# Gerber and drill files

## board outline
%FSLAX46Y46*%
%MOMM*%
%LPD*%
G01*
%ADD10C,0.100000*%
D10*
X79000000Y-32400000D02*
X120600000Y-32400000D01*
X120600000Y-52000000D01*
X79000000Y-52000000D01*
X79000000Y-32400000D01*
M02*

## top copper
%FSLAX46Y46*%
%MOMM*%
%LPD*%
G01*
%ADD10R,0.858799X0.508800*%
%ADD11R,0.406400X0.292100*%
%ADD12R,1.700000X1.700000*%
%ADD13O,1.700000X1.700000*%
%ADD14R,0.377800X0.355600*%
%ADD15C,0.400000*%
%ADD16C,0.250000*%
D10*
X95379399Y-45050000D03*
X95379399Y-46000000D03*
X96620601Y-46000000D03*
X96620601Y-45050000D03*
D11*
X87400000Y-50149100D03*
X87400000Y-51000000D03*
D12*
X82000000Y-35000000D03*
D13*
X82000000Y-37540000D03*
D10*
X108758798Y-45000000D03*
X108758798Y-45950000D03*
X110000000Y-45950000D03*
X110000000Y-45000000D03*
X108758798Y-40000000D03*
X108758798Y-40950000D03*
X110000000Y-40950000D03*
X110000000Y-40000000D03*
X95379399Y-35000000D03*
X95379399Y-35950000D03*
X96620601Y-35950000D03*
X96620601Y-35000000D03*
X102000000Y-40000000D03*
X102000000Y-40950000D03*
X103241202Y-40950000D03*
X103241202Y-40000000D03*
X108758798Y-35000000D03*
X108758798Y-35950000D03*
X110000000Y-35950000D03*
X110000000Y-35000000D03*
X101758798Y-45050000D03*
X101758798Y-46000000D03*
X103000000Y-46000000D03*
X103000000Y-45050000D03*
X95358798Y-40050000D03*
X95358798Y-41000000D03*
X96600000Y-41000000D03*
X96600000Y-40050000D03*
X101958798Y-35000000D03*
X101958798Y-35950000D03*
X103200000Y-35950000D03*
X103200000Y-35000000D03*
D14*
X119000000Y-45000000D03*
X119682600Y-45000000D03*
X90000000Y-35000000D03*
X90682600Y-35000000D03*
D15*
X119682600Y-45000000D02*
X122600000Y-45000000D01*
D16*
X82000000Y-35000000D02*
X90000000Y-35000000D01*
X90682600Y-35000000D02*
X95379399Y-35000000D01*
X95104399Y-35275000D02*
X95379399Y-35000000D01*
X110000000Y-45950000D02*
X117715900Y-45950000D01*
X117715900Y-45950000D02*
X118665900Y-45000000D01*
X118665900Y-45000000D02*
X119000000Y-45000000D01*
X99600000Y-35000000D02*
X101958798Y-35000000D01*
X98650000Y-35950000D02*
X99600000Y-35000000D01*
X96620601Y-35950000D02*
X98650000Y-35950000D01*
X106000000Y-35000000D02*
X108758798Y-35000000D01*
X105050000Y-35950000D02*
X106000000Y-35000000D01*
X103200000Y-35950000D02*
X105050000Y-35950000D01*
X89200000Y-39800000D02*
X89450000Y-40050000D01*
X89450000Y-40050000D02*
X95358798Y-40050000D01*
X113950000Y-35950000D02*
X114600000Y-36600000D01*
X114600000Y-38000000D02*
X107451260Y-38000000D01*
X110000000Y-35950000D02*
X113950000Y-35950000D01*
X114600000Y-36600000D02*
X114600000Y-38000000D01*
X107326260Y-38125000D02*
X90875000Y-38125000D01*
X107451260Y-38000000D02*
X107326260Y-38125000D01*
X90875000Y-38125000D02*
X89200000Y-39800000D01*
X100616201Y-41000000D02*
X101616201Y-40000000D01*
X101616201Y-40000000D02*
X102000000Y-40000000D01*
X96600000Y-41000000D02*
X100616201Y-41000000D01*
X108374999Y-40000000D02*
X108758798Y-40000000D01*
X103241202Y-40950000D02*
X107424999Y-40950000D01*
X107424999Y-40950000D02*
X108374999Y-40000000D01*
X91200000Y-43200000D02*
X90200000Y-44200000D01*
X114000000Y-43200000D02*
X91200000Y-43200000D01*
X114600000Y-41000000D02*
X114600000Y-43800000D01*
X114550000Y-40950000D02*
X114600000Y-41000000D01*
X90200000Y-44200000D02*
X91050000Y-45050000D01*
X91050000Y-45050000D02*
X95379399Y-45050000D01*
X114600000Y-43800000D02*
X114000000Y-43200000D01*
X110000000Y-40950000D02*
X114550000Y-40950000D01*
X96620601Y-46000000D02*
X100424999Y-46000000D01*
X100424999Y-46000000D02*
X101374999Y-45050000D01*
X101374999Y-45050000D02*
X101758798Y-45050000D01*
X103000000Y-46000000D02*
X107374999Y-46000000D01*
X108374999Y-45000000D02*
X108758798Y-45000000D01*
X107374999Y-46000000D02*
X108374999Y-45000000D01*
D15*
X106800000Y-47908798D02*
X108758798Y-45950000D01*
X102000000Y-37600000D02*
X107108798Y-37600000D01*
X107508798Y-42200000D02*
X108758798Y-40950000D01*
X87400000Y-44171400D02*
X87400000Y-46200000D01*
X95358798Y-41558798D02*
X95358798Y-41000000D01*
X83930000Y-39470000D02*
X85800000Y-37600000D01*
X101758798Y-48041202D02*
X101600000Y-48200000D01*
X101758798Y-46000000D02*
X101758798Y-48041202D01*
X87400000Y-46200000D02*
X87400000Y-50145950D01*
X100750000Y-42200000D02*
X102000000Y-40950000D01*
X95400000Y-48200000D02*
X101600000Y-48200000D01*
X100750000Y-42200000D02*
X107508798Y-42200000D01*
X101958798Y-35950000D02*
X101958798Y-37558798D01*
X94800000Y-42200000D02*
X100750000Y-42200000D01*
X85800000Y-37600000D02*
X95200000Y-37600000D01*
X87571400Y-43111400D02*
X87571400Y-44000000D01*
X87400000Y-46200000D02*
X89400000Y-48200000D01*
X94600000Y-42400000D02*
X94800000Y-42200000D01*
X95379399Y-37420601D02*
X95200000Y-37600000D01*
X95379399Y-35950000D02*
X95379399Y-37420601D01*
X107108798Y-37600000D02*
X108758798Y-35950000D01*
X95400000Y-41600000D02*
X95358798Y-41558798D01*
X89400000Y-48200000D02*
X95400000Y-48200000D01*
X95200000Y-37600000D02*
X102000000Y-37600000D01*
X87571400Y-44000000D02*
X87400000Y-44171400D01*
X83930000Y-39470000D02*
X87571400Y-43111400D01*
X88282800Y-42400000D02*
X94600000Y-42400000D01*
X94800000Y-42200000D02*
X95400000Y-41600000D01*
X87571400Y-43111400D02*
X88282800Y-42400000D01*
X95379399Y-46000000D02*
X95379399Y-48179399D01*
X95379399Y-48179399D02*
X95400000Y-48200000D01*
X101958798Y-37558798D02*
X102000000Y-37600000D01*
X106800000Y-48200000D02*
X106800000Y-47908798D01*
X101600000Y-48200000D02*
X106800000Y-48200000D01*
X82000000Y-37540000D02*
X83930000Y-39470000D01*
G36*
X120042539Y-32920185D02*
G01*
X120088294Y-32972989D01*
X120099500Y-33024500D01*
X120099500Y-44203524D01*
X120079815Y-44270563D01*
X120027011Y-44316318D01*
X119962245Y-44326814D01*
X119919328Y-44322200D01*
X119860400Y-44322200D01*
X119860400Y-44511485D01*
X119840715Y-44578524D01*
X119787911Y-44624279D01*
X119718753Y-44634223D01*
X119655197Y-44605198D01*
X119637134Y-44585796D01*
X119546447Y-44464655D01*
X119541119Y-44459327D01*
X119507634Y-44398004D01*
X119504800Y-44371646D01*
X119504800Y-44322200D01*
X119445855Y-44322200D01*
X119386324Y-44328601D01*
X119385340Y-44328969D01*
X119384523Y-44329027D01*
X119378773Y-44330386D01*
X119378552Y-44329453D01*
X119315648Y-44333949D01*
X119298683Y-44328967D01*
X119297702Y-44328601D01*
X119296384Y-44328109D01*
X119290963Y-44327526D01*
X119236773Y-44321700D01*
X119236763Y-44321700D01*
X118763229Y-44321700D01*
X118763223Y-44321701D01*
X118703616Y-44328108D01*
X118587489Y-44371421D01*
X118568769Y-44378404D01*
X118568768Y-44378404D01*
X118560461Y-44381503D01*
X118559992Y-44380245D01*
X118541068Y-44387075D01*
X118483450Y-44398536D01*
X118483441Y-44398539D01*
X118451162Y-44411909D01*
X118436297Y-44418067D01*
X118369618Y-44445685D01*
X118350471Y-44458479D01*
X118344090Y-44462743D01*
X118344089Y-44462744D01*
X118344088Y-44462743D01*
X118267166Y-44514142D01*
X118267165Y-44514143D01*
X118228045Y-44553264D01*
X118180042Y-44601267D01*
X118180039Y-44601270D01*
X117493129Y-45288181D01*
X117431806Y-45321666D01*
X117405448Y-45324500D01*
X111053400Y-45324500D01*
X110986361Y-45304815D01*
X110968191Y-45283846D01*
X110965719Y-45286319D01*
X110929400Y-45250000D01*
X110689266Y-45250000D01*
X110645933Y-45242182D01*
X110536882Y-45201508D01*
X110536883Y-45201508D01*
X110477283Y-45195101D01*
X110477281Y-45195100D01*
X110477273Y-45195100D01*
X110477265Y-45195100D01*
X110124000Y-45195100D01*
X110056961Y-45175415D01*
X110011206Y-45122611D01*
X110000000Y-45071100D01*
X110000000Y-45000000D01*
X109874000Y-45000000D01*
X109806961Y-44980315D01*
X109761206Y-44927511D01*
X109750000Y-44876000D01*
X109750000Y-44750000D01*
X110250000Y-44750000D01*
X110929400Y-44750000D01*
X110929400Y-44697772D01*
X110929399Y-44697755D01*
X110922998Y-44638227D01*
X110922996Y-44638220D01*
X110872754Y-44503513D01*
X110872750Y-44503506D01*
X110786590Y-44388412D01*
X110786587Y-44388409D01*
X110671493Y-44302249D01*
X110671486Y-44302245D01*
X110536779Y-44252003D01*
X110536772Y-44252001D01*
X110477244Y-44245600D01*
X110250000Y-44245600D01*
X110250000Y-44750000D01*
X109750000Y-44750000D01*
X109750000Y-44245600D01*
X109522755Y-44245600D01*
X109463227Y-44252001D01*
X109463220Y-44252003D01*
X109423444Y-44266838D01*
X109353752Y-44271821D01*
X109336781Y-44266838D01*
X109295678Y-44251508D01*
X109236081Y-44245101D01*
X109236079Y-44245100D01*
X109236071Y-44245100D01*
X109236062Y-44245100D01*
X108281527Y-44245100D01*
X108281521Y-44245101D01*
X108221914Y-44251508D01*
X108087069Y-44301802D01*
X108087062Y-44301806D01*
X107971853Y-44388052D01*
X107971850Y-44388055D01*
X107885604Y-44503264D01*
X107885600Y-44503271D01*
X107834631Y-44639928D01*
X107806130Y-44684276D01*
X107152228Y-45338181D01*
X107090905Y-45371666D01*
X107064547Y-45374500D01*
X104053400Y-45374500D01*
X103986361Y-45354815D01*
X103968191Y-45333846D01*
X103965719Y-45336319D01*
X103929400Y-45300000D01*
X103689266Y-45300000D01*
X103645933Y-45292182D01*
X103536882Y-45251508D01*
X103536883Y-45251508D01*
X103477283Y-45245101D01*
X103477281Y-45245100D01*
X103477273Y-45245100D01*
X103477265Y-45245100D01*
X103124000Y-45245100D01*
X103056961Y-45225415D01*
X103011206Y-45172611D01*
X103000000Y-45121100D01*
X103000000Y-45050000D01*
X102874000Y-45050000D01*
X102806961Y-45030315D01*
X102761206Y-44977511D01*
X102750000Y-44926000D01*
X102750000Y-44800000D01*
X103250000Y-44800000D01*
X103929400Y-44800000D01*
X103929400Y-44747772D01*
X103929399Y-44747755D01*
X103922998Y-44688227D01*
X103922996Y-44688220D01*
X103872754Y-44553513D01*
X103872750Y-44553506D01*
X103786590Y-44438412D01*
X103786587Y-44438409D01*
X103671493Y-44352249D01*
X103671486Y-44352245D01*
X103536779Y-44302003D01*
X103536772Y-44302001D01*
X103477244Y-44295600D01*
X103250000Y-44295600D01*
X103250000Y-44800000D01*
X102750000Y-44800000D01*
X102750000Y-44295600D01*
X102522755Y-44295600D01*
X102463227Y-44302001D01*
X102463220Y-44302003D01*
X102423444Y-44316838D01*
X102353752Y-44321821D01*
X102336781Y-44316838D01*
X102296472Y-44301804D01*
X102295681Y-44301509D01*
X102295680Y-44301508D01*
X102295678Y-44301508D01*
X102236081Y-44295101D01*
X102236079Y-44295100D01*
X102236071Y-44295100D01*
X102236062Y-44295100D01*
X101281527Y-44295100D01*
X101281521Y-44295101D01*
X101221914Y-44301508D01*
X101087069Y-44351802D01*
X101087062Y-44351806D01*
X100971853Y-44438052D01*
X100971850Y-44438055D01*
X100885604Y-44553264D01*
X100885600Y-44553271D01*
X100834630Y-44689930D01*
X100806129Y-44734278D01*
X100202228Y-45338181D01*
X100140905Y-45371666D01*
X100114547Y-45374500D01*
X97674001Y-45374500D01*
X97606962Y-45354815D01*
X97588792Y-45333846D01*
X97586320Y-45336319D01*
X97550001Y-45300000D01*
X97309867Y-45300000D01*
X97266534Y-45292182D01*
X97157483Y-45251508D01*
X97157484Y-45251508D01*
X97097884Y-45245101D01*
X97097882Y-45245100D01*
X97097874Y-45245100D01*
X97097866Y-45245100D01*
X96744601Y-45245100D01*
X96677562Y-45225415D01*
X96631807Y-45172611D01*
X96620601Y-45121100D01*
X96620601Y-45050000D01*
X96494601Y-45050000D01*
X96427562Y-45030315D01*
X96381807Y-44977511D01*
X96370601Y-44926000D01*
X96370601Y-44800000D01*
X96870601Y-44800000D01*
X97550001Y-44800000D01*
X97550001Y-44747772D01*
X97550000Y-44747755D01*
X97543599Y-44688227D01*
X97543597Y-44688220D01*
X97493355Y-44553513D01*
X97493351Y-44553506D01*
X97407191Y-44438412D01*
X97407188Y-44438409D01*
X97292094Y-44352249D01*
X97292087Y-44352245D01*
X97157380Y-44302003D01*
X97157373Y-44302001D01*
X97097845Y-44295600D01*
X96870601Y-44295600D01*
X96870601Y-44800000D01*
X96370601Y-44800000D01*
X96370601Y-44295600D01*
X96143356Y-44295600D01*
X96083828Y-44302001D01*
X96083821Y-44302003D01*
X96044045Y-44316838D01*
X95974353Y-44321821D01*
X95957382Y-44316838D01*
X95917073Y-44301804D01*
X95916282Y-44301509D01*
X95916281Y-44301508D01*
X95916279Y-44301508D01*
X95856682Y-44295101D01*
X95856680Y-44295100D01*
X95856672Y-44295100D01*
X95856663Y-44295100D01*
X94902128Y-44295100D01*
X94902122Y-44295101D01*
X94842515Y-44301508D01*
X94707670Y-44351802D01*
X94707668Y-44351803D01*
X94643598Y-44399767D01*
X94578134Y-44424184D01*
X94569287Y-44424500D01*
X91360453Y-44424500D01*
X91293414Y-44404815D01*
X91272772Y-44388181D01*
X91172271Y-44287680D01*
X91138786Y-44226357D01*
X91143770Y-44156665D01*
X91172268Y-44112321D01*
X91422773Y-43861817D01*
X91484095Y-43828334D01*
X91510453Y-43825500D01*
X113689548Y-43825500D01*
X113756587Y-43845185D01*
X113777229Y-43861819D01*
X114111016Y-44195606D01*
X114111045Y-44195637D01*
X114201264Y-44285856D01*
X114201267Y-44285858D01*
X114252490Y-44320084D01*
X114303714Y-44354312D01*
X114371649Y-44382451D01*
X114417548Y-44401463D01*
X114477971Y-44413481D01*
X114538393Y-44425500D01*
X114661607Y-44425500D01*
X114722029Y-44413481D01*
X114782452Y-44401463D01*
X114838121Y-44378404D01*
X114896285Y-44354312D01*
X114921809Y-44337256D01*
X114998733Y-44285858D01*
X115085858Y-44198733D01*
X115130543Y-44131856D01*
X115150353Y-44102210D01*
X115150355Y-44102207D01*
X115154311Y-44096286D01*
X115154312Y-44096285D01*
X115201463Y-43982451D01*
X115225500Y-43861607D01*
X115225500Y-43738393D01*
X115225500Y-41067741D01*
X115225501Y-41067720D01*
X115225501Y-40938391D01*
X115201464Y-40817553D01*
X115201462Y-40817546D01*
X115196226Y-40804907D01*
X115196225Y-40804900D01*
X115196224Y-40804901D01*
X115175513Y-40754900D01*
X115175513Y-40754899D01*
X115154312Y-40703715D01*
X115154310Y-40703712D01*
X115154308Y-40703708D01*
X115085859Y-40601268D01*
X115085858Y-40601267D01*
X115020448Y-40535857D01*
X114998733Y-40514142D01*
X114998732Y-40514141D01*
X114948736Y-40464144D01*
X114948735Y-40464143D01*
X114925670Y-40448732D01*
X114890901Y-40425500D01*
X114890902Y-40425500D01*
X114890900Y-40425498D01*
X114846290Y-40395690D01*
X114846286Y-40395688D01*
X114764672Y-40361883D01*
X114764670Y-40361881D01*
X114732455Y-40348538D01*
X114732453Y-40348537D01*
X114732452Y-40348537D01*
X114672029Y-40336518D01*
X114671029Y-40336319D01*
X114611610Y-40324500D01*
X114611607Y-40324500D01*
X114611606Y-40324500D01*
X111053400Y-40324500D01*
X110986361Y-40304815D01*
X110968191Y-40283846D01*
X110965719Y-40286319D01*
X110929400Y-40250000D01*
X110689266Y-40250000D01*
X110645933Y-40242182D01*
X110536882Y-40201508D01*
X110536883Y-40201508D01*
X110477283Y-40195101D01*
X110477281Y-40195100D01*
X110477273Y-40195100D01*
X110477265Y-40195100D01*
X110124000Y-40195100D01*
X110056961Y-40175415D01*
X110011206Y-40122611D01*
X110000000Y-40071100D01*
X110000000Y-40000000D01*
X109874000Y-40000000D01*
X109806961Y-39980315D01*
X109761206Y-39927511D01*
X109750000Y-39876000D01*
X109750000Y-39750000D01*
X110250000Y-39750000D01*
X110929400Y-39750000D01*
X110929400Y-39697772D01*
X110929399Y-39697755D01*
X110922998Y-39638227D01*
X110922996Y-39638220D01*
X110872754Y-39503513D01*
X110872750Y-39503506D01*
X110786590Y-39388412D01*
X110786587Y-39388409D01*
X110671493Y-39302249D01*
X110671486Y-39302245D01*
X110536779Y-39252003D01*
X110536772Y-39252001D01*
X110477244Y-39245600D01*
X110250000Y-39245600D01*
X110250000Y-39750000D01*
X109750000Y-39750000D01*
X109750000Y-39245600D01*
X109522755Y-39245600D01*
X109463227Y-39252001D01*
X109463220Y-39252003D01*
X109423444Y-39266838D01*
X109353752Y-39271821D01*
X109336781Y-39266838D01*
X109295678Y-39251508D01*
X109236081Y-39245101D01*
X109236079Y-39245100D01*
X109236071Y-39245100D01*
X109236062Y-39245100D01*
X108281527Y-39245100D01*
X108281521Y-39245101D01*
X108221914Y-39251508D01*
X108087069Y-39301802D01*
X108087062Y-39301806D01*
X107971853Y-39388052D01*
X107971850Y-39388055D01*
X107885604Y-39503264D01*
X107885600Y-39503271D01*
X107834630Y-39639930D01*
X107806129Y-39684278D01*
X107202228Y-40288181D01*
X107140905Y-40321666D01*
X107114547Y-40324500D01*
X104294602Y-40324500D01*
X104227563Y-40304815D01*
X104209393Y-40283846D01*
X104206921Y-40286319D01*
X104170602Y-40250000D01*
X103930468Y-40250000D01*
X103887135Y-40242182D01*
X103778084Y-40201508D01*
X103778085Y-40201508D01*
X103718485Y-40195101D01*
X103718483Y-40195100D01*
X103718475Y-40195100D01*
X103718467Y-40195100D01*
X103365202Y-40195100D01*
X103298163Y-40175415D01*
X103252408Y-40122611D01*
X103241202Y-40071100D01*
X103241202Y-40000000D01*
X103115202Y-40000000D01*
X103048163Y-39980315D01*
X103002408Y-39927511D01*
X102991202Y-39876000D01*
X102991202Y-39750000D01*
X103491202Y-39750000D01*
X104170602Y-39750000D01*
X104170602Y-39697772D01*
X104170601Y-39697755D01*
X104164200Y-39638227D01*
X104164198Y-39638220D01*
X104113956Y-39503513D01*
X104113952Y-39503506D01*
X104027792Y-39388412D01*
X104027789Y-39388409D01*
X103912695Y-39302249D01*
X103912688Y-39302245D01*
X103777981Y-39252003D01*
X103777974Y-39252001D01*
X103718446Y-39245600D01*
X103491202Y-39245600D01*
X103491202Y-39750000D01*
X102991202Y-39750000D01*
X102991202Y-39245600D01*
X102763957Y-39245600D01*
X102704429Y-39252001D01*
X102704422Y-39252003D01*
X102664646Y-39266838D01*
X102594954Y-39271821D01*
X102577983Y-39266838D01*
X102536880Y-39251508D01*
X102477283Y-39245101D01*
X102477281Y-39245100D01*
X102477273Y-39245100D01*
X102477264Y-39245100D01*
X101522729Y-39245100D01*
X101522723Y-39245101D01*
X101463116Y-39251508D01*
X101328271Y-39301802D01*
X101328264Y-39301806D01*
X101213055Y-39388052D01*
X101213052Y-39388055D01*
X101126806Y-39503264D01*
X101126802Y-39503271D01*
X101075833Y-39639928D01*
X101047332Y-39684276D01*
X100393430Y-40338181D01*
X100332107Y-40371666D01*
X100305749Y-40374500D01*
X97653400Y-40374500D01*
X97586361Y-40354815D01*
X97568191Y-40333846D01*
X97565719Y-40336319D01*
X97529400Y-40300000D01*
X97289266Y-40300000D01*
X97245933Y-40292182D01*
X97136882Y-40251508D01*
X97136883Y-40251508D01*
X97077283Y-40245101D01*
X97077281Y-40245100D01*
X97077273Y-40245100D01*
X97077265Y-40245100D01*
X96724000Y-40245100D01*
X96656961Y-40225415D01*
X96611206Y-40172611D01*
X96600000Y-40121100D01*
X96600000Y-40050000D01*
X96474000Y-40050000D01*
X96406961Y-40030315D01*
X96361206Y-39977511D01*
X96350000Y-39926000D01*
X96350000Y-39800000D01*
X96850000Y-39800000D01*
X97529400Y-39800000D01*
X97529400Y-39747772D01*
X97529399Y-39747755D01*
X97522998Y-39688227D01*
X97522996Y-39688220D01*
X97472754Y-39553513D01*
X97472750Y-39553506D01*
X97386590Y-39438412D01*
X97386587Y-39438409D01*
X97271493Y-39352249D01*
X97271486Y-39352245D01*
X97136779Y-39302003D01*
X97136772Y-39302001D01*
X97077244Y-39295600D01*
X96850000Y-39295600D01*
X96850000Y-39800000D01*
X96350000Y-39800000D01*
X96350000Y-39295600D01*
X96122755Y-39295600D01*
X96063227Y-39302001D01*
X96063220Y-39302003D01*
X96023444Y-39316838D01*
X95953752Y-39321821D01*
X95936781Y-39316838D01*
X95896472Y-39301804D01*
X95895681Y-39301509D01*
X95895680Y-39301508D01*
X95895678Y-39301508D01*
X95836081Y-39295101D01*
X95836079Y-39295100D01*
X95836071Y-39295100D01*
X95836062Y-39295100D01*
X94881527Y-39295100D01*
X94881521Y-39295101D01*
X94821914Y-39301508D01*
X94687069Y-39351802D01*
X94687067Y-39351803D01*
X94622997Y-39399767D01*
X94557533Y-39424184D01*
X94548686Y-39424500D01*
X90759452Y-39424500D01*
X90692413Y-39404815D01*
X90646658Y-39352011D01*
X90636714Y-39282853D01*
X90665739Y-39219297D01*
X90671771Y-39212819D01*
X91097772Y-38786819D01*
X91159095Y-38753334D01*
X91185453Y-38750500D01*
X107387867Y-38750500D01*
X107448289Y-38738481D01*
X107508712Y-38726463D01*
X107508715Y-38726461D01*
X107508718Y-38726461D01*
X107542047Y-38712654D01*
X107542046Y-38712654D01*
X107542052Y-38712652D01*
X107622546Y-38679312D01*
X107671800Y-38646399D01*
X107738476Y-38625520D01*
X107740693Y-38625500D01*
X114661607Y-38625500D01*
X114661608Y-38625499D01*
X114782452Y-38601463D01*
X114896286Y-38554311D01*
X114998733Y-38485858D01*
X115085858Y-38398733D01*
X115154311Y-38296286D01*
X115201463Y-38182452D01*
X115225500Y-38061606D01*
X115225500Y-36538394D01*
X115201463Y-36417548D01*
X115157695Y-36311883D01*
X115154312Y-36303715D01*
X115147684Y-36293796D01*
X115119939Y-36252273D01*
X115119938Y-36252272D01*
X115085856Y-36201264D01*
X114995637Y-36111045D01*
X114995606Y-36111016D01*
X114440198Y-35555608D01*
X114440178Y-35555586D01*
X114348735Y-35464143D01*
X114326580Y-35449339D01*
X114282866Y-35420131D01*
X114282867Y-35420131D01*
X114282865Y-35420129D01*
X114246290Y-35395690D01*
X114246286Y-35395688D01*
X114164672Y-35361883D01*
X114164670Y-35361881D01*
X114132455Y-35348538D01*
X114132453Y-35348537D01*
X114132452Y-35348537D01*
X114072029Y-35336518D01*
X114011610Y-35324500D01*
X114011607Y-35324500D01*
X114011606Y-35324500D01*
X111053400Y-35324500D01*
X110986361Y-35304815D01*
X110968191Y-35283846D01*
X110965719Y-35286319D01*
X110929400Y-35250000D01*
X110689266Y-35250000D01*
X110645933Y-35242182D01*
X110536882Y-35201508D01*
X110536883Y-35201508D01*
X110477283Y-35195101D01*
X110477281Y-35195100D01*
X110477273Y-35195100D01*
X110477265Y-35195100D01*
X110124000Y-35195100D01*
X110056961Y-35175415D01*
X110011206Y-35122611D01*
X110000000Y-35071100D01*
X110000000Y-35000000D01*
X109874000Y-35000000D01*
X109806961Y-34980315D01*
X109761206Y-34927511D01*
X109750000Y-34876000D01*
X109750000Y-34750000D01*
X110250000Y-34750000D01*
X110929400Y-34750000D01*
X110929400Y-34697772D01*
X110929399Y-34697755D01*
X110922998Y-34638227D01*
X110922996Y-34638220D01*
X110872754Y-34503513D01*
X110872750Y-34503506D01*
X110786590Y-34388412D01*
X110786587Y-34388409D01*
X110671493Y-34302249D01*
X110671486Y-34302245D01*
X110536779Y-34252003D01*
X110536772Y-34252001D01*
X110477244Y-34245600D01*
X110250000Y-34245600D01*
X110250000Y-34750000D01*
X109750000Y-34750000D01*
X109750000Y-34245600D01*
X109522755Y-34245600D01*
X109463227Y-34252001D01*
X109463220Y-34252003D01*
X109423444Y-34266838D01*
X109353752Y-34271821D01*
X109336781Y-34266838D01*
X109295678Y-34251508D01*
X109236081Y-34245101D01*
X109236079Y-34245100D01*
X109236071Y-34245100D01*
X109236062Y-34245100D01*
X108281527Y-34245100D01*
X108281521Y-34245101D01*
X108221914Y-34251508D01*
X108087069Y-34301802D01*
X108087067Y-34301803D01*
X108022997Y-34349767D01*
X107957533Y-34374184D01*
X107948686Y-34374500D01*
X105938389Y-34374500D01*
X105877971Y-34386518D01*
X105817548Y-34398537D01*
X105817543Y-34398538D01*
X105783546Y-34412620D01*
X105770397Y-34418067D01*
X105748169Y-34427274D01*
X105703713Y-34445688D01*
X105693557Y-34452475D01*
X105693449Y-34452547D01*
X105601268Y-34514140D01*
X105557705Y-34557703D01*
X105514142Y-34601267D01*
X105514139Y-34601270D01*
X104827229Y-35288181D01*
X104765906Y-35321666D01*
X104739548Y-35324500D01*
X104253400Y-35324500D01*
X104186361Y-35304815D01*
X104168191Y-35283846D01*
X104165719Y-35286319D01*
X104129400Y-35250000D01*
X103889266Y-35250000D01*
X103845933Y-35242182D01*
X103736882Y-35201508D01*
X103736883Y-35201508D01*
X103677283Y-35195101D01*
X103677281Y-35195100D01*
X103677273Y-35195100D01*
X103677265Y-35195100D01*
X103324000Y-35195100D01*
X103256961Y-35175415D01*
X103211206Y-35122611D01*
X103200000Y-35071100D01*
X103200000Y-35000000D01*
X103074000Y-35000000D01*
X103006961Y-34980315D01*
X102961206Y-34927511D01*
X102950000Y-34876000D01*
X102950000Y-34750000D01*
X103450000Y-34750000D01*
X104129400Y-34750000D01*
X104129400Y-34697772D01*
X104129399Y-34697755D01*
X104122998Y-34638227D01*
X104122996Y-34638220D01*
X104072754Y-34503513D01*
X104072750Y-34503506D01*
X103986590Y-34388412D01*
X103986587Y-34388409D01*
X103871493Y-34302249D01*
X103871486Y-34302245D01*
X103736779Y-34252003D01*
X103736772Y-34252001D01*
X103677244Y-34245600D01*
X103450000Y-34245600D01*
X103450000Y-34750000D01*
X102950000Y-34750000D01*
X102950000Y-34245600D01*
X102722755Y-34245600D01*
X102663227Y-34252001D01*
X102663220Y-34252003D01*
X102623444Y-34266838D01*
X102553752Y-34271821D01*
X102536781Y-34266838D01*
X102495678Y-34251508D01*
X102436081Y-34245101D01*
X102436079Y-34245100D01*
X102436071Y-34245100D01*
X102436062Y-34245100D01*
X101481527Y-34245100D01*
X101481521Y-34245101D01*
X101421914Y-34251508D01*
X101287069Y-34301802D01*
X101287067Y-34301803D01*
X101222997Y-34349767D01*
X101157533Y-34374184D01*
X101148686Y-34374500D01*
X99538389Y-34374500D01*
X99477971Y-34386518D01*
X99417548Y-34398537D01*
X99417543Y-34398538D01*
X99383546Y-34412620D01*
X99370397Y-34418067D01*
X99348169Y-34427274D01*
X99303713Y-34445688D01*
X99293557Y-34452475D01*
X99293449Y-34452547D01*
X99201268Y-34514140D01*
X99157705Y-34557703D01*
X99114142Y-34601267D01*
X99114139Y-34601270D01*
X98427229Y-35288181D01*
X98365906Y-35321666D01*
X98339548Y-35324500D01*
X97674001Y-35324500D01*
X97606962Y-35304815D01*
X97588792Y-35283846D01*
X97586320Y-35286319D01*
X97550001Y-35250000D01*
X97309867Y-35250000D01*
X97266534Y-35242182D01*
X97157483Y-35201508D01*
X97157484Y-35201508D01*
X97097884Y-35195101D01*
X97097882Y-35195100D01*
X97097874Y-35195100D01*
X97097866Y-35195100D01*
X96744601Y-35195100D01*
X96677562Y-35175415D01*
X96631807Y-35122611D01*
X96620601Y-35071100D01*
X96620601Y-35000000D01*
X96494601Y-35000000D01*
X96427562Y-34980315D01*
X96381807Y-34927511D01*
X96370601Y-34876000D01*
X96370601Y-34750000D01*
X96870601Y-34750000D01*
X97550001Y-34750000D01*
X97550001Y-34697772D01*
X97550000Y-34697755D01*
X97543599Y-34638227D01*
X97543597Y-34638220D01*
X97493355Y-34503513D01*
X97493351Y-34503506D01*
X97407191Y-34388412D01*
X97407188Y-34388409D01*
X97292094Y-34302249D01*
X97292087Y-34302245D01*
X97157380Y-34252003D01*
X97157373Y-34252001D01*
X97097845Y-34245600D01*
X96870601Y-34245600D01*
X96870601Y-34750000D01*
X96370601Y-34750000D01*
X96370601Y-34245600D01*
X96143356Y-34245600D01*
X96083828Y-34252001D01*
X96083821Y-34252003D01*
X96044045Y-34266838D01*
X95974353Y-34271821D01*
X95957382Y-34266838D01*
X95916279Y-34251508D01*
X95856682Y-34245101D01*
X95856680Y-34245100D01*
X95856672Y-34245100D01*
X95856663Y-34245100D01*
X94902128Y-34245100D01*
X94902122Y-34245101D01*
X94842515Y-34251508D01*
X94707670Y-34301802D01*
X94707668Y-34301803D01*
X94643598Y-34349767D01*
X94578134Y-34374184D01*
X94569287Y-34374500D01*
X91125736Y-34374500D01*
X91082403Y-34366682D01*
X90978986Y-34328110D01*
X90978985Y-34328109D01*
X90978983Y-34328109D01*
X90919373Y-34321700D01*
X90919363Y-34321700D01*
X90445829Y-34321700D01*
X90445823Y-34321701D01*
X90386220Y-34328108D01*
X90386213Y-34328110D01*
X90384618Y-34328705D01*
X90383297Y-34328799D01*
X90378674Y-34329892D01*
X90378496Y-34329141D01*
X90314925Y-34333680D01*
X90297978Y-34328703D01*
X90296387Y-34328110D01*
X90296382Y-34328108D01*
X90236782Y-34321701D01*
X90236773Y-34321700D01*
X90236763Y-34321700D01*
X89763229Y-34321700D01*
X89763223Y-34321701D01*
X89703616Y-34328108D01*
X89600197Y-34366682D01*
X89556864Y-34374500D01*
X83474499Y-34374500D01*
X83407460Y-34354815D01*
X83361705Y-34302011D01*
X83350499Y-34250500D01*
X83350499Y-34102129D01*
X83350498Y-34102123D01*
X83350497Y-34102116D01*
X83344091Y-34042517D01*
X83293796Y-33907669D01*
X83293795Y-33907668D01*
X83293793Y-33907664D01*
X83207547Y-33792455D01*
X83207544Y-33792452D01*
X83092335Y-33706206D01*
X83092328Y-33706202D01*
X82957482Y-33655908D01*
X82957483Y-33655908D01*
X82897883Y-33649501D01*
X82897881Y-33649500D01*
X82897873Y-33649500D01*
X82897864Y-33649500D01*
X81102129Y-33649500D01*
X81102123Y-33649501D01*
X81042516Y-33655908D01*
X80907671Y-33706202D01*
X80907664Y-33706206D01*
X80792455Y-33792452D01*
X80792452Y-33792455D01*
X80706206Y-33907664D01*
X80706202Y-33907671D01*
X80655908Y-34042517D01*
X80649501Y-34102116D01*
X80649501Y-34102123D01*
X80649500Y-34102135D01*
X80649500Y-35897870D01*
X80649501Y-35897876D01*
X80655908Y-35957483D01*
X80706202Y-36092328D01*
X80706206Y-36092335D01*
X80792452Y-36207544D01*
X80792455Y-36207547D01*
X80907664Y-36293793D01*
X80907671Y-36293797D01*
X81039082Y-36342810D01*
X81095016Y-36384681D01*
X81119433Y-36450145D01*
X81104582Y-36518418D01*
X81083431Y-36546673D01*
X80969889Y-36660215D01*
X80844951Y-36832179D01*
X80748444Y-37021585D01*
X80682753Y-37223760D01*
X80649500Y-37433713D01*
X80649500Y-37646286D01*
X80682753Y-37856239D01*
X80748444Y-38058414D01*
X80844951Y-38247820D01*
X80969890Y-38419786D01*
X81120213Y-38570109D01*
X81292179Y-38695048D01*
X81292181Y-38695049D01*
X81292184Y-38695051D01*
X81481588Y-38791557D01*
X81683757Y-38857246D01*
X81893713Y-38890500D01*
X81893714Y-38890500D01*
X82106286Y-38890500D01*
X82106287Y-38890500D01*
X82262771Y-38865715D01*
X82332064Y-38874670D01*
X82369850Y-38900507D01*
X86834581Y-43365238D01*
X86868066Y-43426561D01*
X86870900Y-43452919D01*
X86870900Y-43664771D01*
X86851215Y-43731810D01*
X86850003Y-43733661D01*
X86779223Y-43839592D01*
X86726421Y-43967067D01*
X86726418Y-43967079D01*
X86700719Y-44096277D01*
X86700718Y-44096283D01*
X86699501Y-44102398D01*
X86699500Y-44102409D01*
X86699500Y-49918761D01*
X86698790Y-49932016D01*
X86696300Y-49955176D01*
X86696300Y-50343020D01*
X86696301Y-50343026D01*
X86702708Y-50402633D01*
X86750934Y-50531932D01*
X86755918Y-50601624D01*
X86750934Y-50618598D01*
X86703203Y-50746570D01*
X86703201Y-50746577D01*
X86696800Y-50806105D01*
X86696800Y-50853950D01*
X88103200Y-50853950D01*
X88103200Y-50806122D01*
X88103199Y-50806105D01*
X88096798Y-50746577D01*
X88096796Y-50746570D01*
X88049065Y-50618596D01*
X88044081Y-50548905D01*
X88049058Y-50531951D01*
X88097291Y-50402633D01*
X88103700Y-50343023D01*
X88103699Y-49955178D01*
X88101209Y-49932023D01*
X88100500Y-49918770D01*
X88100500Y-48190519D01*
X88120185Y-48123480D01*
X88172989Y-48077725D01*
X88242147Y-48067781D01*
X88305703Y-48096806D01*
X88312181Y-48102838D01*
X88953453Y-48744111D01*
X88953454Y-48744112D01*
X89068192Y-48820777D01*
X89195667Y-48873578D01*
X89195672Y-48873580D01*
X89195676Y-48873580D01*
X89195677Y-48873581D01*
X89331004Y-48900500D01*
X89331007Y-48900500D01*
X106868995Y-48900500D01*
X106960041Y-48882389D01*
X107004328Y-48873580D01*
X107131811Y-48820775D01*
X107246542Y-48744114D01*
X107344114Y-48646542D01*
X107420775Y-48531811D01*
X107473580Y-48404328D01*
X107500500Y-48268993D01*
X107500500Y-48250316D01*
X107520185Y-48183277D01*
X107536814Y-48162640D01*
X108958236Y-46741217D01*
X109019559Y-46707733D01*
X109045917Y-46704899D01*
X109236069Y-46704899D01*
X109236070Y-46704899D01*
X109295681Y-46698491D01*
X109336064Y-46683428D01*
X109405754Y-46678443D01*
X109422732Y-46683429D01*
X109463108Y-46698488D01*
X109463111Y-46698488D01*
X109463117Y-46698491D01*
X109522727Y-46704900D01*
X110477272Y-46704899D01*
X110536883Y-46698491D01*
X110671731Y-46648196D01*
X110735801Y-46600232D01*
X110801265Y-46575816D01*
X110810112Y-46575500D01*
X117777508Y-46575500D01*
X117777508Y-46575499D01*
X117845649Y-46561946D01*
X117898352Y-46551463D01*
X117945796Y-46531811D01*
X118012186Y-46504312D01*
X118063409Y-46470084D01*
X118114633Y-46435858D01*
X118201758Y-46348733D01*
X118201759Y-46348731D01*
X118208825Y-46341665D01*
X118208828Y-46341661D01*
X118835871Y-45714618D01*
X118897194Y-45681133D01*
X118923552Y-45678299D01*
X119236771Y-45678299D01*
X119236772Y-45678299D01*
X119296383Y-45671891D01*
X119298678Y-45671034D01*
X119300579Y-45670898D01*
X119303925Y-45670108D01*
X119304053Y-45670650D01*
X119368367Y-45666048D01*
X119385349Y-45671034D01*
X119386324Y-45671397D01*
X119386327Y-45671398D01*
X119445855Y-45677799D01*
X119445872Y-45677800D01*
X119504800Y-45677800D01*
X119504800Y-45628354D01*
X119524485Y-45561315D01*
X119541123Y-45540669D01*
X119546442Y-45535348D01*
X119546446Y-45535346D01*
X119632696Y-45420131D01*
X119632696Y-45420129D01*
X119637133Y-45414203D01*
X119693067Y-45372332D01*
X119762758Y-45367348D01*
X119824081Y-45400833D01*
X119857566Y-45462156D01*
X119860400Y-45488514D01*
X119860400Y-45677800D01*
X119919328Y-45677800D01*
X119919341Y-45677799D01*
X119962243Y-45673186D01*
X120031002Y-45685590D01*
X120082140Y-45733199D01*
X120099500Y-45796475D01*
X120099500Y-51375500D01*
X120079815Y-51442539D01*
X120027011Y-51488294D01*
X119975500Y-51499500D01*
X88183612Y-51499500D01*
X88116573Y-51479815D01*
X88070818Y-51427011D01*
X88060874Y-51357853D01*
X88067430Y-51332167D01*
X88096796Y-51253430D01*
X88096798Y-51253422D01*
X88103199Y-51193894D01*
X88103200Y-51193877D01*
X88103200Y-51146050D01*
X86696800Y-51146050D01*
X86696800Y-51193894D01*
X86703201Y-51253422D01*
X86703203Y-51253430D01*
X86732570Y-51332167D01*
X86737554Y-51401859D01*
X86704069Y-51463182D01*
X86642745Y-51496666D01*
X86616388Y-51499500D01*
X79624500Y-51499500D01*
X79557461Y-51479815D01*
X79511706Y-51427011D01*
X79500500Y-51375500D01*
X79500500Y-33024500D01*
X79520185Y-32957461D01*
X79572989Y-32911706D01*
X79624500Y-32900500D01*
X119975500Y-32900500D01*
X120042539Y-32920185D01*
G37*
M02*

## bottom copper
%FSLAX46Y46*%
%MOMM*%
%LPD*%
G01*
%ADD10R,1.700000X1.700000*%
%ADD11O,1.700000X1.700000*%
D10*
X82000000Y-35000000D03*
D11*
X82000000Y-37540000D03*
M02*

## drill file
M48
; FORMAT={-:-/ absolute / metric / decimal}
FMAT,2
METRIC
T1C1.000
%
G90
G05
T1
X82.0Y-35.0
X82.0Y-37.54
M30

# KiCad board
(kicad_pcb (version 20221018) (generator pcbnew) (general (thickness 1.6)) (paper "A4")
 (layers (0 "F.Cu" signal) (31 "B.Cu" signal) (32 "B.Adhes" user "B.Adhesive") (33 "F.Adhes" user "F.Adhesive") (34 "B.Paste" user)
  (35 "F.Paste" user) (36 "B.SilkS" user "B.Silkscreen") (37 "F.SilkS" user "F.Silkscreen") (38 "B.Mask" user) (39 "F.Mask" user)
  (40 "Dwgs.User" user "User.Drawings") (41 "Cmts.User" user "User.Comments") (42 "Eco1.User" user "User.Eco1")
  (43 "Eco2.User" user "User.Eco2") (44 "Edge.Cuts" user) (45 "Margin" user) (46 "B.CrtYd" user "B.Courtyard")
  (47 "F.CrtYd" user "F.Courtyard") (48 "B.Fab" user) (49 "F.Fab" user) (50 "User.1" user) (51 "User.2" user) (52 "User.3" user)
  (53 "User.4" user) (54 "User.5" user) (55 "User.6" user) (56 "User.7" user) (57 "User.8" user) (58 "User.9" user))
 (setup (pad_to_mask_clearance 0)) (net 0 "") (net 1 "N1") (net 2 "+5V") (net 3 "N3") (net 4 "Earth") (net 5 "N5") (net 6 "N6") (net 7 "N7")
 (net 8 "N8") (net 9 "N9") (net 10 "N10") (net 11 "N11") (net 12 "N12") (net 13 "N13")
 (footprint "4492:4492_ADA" (layer "F.Cu") (at 96 45.525)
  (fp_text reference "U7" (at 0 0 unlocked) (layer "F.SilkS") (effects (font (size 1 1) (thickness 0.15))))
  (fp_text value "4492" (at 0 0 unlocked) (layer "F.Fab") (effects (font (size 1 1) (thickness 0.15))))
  (pad "1" smd rect (at -0.620601 -0.475) (size 0.858799 0.5088) (layers "F.Cu" "F.Paste" "F.Mask") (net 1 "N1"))
  (pad "2" smd rect (at -0.620601 0.475) (size 0.858799 0.5088) (layers "F.Cu" "F.Paste" "F.Mask") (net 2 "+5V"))
  (pad "3" smd rect (at 0.620601 0.475) (size 0.858799 0.5088) (layers "F.Cu" "F.Paste" "F.Mask") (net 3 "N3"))
  (pad "4" smd rect (at 0.620601 -0.475) (size 0.858799 0.5088) (layers "F.Cu" "F.Paste" "F.Mask") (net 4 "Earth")))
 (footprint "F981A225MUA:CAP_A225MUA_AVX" (layer "F.Cu") (at 87.4 50.57455 -90)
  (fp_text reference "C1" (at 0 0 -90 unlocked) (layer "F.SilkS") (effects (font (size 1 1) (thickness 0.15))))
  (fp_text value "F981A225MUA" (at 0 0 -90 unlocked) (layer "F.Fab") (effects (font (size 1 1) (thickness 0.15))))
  (pad "1" smd rect (at -0.42545 0 270) (size 0.2921 0.4064) (layers "F.Cu" "F.Paste" "F.Mask") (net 2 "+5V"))
  (pad "2" smd rect (at 0.42545 0 270) (size 0.2921 0.4064) (layers "F.Cu" "F.Paste" "F.Mask") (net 4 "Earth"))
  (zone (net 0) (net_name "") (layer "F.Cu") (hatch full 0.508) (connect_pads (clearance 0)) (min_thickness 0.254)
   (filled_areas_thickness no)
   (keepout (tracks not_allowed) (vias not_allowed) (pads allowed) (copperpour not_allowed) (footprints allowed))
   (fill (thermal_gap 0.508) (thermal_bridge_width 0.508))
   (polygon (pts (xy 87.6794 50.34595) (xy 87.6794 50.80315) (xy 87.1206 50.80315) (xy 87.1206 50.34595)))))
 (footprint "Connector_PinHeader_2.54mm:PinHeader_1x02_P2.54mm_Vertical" (layer "F.Cu") (at 82 35)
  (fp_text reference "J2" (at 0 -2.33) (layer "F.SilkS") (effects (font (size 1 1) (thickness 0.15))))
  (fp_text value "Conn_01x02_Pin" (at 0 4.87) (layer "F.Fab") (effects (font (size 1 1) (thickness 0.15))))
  (pad "1" thru_hole rect (at 0 0) (size 1.7 1.7) (drill 1) (layers "*.Cu" "*.Mask") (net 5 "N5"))
  (pad "2" thru_hole oval (at 0 2.54) (size 1.7 1.7) (drill 1) (layers "*.Cu" "*.Mask") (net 2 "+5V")))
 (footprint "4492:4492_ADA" (layer "F.Cu") (at 109.379399 45.475)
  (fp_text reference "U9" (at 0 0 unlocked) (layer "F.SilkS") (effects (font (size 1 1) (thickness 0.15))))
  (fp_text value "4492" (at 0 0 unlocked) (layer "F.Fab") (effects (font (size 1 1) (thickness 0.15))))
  (pad "1" smd rect (at -0.620601 -0.475) (size 0.858799 0.5088) (layers "F.Cu" "F.Paste" "F.Mask") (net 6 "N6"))
  (pad "2" smd rect (at -0.620601 0.475) (size 0.858799 0.5088) (layers "F.Cu" "F.Paste" "F.Mask") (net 2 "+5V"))
  (pad "3" smd rect (at 0.620601 0.475) (size 0.858799 0.5088) (layers "F.Cu" "F.Paste" "F.Mask") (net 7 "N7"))
  (pad "4" smd rect (at 0.620601 -0.475) (size 0.858799 0.5088) (layers "F.Cu" "F.Paste" "F.Mask") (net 4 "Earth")))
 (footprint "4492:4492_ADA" (layer "F.Cu") (at 109.379399 40.475)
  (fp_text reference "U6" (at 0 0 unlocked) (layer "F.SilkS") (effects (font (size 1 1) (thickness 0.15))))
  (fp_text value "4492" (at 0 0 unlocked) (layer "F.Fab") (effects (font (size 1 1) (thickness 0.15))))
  (pad "1" smd rect (at -0.620601 -0.475) (size 0.858799 0.5088) (layers "F.Cu" "F.Paste" "F.Mask") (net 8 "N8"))
  (pad "2" smd rect (at -0.620601 0.475) (size 0.858799 0.5088) (layers "F.Cu" "F.Paste" "F.Mask") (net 2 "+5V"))
  (pad "3" smd rect (at 0.620601 0.475) (size 0.858799 0.5088) (layers "F.Cu" "F.Paste" "F.Mask") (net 1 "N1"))
  (pad "4" smd rect (at 0.620601 -0.475) (size 0.858799 0.5088) (layers "F.Cu" "F.Paste" "F.Mask") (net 4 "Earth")))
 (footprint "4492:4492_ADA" (layer "F.Cu") (at 96 35.475)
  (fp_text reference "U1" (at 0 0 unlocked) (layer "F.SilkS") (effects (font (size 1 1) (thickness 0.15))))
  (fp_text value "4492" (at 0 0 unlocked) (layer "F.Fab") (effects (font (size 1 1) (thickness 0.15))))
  (pad "1" smd rect (at -0.620601 -0.475) (size 0.858799 0.5088) (layers "F.Cu" "F.Paste" "F.Mask") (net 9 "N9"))
  (pad "2" smd rect (at -0.620601 0.475) (size 0.858799 0.5088) (layers "F.Cu" "F.Paste" "F.Mask") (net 2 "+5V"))
  (pad "3" smd rect (at 0.620601 0.475) (size 0.858799 0.5088) (layers "F.Cu" "F.Paste" "F.Mask") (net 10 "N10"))
  (pad "4" smd rect (at 0.620601 -0.475) (size 0.858799 0.5088) (layers "F.Cu" "F.Paste" "F.Mask") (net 4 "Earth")))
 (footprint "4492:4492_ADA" (layer "F.Cu") (at 102.620601 40.475)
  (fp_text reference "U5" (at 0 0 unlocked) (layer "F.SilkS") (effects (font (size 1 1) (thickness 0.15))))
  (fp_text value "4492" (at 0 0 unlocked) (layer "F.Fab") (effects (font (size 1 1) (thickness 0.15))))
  (pad "1" smd rect (at -0.620601 -0.475) (size 0.858799 0.5088) (layers "F.Cu" "F.Paste" "F.Mask") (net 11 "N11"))
  (pad "2" smd rect (at -0.620601 0.475) (size 0.858799 0.5088) (layers "F.Cu" "F.Paste" "F.Mask") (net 2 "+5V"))
  (pad "3" smd rect (at 0.620601 0.475) (size 0.858799 0.5088) (layers "F.Cu" "F.Paste" "F.Mask") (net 8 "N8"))
  (pad "4" smd rect (at 0.620601 -0.475) (size 0.858799 0.5088) (layers "F.Cu" "F.Paste" "F.Mask") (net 4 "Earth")))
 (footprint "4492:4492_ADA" (layer "F.Cu") (at 109.379399 35.475)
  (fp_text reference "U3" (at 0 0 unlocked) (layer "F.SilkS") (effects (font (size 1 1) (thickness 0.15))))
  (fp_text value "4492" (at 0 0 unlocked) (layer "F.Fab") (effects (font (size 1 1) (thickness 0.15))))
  (pad "1" smd rect (at -0.620601 -0.475) (size 0.858799 0.5088) (layers "F.Cu" "F.Paste" "F.Mask") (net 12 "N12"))
  (pad "2" smd rect (at -0.620601 0.475) (size 0.858799 0.5088) (layers "F.Cu" "F.Paste" "F.Mask") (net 2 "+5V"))
  (pad "3" smd rect (at 0.620601 0.475) (size 0.858799 0.5088) (layers "F.Cu" "F.Paste" "F.Mask") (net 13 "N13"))
  (pad "4" smd rect (at 0.620601 -0.475) (size 0.858799 0.5088) (layers "F.Cu" "F.Paste" "F.Mask") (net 4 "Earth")))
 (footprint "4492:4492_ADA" (layer "F.Cu") (at 102.379399 45.525)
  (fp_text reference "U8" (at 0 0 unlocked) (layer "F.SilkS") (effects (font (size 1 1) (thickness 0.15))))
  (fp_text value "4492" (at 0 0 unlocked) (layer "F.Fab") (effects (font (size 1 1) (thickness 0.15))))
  (pad "1" smd rect (at -0.620601 -0.475) (size 0.858799 0.5088) (layers "F.Cu" "F.Paste" "F.Mask") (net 3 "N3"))
  (pad "2" smd rect (at -0.620601 0.475) (size 0.858799 0.5088) (layers "F.Cu" "F.Paste" "F.Mask") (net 2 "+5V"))
  (pad "3" smd rect (at 0.620601 0.475) (size 0.858799 0.5088) (layers "F.Cu" "F.Paste" "F.Mask") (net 6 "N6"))
  (pad "4" smd rect (at 0.620601 -0.475) (size 0.858799 0.5088) (layers "F.Cu" "F.Paste" "F.Mask") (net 4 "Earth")))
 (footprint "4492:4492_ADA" (layer "F.Cu") (at 95.979399 40.525)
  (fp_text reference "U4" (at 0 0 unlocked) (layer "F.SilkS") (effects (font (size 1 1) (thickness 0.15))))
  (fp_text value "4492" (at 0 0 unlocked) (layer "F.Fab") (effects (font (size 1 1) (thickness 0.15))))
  (pad "1" smd rect (at -0.620601 -0.475) (size 0.858799 0.5088) (layers "F.Cu" "F.Paste" "F.Mask") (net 13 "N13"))
  (pad "2" smd rect (at -0.620601 0.475) (size 0.858799 0.5088) (layers "F.Cu" "F.Paste" "F.Mask") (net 2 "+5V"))
  (pad "3" smd rect (at 0.620601 0.475) (size 0.858799 0.5088) (layers "F.Cu" "F.Paste" "F.Mask") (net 11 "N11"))
  (pad "4" smd rect (at 0.620601 -0.475) (size 0.858799 0.5088) (layers "F.Cu" "F.Paste" "F.Mask") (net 4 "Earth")))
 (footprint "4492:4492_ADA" (layer "F.Cu") (at 102.579399 35.475)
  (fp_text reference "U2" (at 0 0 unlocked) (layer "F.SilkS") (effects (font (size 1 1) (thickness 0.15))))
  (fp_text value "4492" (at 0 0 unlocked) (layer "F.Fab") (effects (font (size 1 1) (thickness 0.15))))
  (pad "1" smd rect (at -0.620601 -0.475) (size 0.858799 0.5088) (layers "F.Cu" "F.Paste" "F.Mask") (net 10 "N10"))
  (pad "2" smd rect (at -0.620601 0.475) (size 0.858799 0.5088) (layers "F.Cu" "F.Paste" "F.Mask") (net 2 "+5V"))
  (pad "3" smd rect (at 0.620601 0.475) (size 0.858799 0.5088) (layers "F.Cu" "F.Paste" "F.Mask") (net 12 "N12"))
  (pad "4" smd rect (at 0.620601 -0.475) (size 0.858799 0.5088) (layers "F.Cu" "F.Paste" "F.Mask") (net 4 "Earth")))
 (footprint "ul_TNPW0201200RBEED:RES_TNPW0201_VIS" (layer "F.Cu") (at 119.3413 45)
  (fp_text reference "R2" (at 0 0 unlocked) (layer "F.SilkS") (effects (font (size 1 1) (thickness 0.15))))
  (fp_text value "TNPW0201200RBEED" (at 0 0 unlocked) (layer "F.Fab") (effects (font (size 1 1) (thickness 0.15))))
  (pad "1" smd rect (at -0.3413 0) (size 0.3778 0.3556) (layers "F.Cu" "F.Paste" "F.Mask") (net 7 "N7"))
  (pad "2" smd rect (at 0.3413 0) (size 0.3778 0.3556) (layers "F.Cu" "F.Paste" "F.Mask") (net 4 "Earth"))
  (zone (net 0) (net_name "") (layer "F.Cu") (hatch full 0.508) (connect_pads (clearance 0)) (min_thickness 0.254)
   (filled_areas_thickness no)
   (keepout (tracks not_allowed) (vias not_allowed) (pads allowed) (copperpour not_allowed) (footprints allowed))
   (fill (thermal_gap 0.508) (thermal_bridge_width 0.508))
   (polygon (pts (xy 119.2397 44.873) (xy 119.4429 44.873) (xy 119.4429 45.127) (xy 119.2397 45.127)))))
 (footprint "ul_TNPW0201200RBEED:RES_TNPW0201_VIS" (layer "F.Cu") (at 90.3413 35)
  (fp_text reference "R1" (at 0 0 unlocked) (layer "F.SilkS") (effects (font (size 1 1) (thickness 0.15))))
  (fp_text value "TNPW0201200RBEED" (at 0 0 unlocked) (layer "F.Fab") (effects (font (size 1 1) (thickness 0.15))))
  (pad "1" smd rect (at -0.3413 0) (size 0.3778 0.3556) (layers "F.Cu" "F.Paste" "F.Mask") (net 5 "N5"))
  (pad "2" smd rect (at 0.3413 0) (size 0.3778 0.3556) (layers "F.Cu" "F.Paste" "F.Mask") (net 9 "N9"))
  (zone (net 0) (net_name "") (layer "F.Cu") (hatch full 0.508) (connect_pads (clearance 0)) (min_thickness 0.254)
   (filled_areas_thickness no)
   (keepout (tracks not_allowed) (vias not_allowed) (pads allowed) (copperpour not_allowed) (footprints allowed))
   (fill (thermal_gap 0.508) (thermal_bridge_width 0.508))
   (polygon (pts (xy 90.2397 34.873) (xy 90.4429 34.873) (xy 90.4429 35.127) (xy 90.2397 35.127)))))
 (gr_rect (start 79 32.4) (end 120.6 52) (stroke (width 0.1) (type default)) (fill none) (layer "Edge.Cuts"))
 (segment (start 119.6826 45) (end 122.6 45) (width 0.4) (layer "F.Cu") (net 4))
 (segment (start 82 35) (end 90 35) (width 0.25) (layer "F.Cu") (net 5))
 (segment (start 90.6826 35) (end 95.379399 35) (width 0.25) (layer "F.Cu") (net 9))
 (segment (start 95.104399 35.275) (end 95.379399 35) (width 0.25) (layer "F.Cu") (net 9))
 (segment (start 110 45.95) (end 117.7159 45.95) (width 0.25) (layer "F.Cu") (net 7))
 (segment (start 117.7159 45.95) (end 118.6659 45) (width 0.25) (layer "F.Cu") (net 7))
 (segment (start 118.6659 45) (end 119 45) (width 0.25) (layer "F.Cu") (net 7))
 (segment (start 99.6 35) (end 101.958798 35) (width 0.25) (layer "F.Cu") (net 10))
 (segment (start 98.65 35.95) (end 99.6 35) (width 0.25) (layer "F.Cu") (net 10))
 (segment (start 96.620601 35.95) (end 98.65 35.95) (width 0.25) (layer "F.Cu") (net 10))
 (segment (start 106 35) (end 108.758798 35) (width 0.25) (layer "F.Cu") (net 12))
 (segment (start 105.05 35.95) (end 106 35) (width 0.25) (layer "F.Cu") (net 12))
 (segment (start 103.2 35.95) (end 105.05 35.95) (width 0.25) (layer "F.Cu") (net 12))
 (segment (start 89.2 39.8) (end 89.45 40.05) (width 0.25) (layer "F.Cu") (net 13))
 (segment (start 89.45 40.05) (end 95.358798 40.05) (width 0.25) (layer "F.Cu") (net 13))
 (segment (start 113.95 35.95) (end 114.6 36.6) (width 0.25) (layer "F.Cu") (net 13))
 (segment (start 114.6 38) (end 107.45126 38) (width 0.25) (layer "F.Cu") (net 13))
 (segment (start 110 35.95) (end 113.95 35.95) (width 0.25) (layer "F.Cu") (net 13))
 (segment (start 114.6 36.6) (end 114.6 38) (width 0.25) (layer "F.Cu") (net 13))
 (segment (start 107.32626 38.125) (end 90.875 38.125) (width 0.25) (layer "F.Cu") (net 13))
 (segment (start 107.45126 38) (end 107.32626 38.125) (width 0.25) (layer "F.Cu") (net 13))
 (segment (start 90.875 38.125) (end 89.2 39.8) (width 0.25) (layer "F.Cu") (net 13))
 (segment (start 100.616201 41) (end 101.616201 40) (width 0.25) (layer "F.Cu") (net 11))
 (segment (start 101.616201 40) (end 102 40) (width 0.25) (layer "F.Cu") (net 11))
 (segment (start 96.6 41) (end 100.616201 41) (width 0.25) (layer "F.Cu") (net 11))
 (segment (start 108.374999 40) (end 108.758798 40) (width 0.25) (layer "F.Cu") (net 8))
 (segment (start 103.241202 40.95) (end 107.424999 40.95) (width 0.25) (layer "F.Cu") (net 8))
 (segment (start 107.424999 40.95) (end 108.374999 40) (width 0.25) (layer "F.Cu") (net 8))
 (segment (start 91.2 43.2) (end 90.2 44.2) (width 0.25) (layer "F.Cu") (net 1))
 (segment (start 114 43.2) (end 91.2 43.2) (width 0.25) (layer "F.Cu") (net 1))
 (segment (start 114.6 41) (end 114.6 43.8) (width 0.25) (layer "F.Cu") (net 1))
 (segment (start 114.55 40.95) (end 114.6 41) (width 0.25) (layer "F.Cu") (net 1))
 (segment (start 90.2 44.2) (end 91.05 45.05) (width 0.25) (layer "F.Cu") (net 1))
 (segment (start 91.05 45.05) (end 95.379399 45.05) (width 0.25) (layer "F.Cu") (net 1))
 (segment (start 114.6 43.8) (end 114 43.2) (width 0.25) (layer "F.Cu") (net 1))
 (segment (start 110 40.95) (end 114.55 40.95) (width 0.25) (layer "F.Cu") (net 1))
 (segment (start 96.620601 46) (end 100.424999 46) (width 0.25) (layer "F.Cu") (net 3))
 (segment (start 100.424999 46) (end 101.374999 45.05) (width 0.25) (layer "F.Cu") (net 3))
 (segment (start 101.374999 45.05) (end 101.758798 45.05) (width 0.25) (layer "F.Cu") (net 3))
 (segment (start 103 46) (end 107.374999 46) (width 0.25) (layer "F.Cu") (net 6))
 (segment (start 108.374999 45) (end 108.758798 45) (width 0.25) (layer "F.Cu") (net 6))
 (segment (start 107.374999 46) (end 108.374999 45) (width 0.25) (layer "F.Cu") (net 6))
 (segment (start 106.8 47.908798) (end 108.758798 45.95) (width 0.4) (layer "F.Cu") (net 2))
 (segment (start 102 37.6) (end 107.108798 37.6) (width 0.4) (layer "F.Cu") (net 2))
 (segment (start 107.508798 42.2) (end 108.758798 40.95) (width 0.4) (layer "F.Cu") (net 2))
 (segment (start 87.4 44.1714) (end 87.4 46.2) (width 0.4) (layer "F.Cu") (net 2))
 (segment (start 95.358798 41.558798) (end 95.358798 41) (width 0.4) (layer "F.Cu") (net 2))
 (segment (start 83.93 39.47) (end 85.8 37.6) (width 0.4) (layer "F.Cu") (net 2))
 (segment (start 101.758798 48.041202) (end 101.6 48.2) (width 0.4) (layer "F.Cu") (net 2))
 (segment (start 101.758798 46) (end 101.758798 48.041202) (width 0.4) (layer "F.Cu") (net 2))
 (segment (start 87.4 46.2) (end 87.4 50.14595) (width 0.4) (layer "F.Cu") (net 2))
 (segment (start 100.75 42.2) (end 102 40.95) (width 0.4) (layer "F.Cu") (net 2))
 (segment (start 95.4 48.2) (end 101.6 48.2) (width 0.4) (layer "F.Cu") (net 2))
 (segment (start 100.75 42.2) (end 107.508798 42.2) (width 0.4) (layer "F.Cu") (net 2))
 (segment (start 101.958798 35.95) (end 101.958798 37.558798) (width 0.4) (layer "F.Cu") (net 2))
 (segment (start 94.8 42.2) (end 100.75 42.2) (width 0.4) (layer "F.Cu") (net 2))
 (segment (start 85.8 37.6) (end 95.2 37.6) (width 0.4) (layer "F.Cu") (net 2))
 (segment (start 87.5714 43.1114) (end 87.5714 44) (width 0.4) (layer "F.Cu") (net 2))
 (segment (start 87.4 46.2) (end 89.4 48.2) (width 0.4) (layer "F.Cu") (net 2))
 (segment (start 94.6 42.4) (end 94.8 42.2) (width 0.4) (layer "F.Cu") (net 2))
 (segment (start 95.379399 37.420601) (end 95.2 37.6) (width 0.4) (layer "F.Cu") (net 2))
 (segment (start 95.379399 35.95) (end 95.379399 37.420601) (width 0.4) (layer "F.Cu") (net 2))
 (segment (start 107.108798 37.6) (end 108.758798 35.95) (width 0.4) (layer "F.Cu") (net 2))
 (segment (start 95.4 41.6) (end 95.358798 41.558798) (width 0.4) (layer "F.Cu") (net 2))
 (segment (start 89.4 48.2) (end 95.4 48.2) (width 0.4) (layer "F.Cu") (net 2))
 (segment (start 95.2 37.6) (end 102 37.6) (width 0.4) (layer "F.Cu") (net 2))
 (segment (start 87.5714 44) (end 87.4 44.1714) (width 0.4) (layer "F.Cu") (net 2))
 (segment (start 83.93 39.47) (end 87.5714 43.1114) (width 0.4) (layer "F.Cu") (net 2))
 (segment (start 88.2828 42.4) (end 94.6 42.4) (width 0.4) (layer "F.Cu") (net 2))
 (segment (start 94.8 42.2) (end 95.4 41.6) (width 0.4) (layer "F.Cu") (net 2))
 (segment (start 87.5714 43.1114) (end 88.2828 42.4) (width 0.4) (layer "F.Cu") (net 2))
 (segment (start 95.379399 46) (end 95.379399 48.179399) (width 0.4) (layer "F.Cu") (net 2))
 (segment (start 95.379399 48.179399) (end 95.4 48.2) (width 0.4) (layer "F.Cu") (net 2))
 (segment (start 101.958798 37.558798) (end 102 37.6) (width 0.4) (layer "F.Cu") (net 2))
 (segment (start 106.8 48.2) (end 106.8 47.908798) (width 0.4) (layer "F.Cu") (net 2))
 (segment (start 101.6 48.2) (end 106.8 48.2) (width 0.4) (layer "F.Cu") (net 2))
 (segment (start 82 37.54) (end 83.93 39.47) (width 0.4) (layer "F.Cu") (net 2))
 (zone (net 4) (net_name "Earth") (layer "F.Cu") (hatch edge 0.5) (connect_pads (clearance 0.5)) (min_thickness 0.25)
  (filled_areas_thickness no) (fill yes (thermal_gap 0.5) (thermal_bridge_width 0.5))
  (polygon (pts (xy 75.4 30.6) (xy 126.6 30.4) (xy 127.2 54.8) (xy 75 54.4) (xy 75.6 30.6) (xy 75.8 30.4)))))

